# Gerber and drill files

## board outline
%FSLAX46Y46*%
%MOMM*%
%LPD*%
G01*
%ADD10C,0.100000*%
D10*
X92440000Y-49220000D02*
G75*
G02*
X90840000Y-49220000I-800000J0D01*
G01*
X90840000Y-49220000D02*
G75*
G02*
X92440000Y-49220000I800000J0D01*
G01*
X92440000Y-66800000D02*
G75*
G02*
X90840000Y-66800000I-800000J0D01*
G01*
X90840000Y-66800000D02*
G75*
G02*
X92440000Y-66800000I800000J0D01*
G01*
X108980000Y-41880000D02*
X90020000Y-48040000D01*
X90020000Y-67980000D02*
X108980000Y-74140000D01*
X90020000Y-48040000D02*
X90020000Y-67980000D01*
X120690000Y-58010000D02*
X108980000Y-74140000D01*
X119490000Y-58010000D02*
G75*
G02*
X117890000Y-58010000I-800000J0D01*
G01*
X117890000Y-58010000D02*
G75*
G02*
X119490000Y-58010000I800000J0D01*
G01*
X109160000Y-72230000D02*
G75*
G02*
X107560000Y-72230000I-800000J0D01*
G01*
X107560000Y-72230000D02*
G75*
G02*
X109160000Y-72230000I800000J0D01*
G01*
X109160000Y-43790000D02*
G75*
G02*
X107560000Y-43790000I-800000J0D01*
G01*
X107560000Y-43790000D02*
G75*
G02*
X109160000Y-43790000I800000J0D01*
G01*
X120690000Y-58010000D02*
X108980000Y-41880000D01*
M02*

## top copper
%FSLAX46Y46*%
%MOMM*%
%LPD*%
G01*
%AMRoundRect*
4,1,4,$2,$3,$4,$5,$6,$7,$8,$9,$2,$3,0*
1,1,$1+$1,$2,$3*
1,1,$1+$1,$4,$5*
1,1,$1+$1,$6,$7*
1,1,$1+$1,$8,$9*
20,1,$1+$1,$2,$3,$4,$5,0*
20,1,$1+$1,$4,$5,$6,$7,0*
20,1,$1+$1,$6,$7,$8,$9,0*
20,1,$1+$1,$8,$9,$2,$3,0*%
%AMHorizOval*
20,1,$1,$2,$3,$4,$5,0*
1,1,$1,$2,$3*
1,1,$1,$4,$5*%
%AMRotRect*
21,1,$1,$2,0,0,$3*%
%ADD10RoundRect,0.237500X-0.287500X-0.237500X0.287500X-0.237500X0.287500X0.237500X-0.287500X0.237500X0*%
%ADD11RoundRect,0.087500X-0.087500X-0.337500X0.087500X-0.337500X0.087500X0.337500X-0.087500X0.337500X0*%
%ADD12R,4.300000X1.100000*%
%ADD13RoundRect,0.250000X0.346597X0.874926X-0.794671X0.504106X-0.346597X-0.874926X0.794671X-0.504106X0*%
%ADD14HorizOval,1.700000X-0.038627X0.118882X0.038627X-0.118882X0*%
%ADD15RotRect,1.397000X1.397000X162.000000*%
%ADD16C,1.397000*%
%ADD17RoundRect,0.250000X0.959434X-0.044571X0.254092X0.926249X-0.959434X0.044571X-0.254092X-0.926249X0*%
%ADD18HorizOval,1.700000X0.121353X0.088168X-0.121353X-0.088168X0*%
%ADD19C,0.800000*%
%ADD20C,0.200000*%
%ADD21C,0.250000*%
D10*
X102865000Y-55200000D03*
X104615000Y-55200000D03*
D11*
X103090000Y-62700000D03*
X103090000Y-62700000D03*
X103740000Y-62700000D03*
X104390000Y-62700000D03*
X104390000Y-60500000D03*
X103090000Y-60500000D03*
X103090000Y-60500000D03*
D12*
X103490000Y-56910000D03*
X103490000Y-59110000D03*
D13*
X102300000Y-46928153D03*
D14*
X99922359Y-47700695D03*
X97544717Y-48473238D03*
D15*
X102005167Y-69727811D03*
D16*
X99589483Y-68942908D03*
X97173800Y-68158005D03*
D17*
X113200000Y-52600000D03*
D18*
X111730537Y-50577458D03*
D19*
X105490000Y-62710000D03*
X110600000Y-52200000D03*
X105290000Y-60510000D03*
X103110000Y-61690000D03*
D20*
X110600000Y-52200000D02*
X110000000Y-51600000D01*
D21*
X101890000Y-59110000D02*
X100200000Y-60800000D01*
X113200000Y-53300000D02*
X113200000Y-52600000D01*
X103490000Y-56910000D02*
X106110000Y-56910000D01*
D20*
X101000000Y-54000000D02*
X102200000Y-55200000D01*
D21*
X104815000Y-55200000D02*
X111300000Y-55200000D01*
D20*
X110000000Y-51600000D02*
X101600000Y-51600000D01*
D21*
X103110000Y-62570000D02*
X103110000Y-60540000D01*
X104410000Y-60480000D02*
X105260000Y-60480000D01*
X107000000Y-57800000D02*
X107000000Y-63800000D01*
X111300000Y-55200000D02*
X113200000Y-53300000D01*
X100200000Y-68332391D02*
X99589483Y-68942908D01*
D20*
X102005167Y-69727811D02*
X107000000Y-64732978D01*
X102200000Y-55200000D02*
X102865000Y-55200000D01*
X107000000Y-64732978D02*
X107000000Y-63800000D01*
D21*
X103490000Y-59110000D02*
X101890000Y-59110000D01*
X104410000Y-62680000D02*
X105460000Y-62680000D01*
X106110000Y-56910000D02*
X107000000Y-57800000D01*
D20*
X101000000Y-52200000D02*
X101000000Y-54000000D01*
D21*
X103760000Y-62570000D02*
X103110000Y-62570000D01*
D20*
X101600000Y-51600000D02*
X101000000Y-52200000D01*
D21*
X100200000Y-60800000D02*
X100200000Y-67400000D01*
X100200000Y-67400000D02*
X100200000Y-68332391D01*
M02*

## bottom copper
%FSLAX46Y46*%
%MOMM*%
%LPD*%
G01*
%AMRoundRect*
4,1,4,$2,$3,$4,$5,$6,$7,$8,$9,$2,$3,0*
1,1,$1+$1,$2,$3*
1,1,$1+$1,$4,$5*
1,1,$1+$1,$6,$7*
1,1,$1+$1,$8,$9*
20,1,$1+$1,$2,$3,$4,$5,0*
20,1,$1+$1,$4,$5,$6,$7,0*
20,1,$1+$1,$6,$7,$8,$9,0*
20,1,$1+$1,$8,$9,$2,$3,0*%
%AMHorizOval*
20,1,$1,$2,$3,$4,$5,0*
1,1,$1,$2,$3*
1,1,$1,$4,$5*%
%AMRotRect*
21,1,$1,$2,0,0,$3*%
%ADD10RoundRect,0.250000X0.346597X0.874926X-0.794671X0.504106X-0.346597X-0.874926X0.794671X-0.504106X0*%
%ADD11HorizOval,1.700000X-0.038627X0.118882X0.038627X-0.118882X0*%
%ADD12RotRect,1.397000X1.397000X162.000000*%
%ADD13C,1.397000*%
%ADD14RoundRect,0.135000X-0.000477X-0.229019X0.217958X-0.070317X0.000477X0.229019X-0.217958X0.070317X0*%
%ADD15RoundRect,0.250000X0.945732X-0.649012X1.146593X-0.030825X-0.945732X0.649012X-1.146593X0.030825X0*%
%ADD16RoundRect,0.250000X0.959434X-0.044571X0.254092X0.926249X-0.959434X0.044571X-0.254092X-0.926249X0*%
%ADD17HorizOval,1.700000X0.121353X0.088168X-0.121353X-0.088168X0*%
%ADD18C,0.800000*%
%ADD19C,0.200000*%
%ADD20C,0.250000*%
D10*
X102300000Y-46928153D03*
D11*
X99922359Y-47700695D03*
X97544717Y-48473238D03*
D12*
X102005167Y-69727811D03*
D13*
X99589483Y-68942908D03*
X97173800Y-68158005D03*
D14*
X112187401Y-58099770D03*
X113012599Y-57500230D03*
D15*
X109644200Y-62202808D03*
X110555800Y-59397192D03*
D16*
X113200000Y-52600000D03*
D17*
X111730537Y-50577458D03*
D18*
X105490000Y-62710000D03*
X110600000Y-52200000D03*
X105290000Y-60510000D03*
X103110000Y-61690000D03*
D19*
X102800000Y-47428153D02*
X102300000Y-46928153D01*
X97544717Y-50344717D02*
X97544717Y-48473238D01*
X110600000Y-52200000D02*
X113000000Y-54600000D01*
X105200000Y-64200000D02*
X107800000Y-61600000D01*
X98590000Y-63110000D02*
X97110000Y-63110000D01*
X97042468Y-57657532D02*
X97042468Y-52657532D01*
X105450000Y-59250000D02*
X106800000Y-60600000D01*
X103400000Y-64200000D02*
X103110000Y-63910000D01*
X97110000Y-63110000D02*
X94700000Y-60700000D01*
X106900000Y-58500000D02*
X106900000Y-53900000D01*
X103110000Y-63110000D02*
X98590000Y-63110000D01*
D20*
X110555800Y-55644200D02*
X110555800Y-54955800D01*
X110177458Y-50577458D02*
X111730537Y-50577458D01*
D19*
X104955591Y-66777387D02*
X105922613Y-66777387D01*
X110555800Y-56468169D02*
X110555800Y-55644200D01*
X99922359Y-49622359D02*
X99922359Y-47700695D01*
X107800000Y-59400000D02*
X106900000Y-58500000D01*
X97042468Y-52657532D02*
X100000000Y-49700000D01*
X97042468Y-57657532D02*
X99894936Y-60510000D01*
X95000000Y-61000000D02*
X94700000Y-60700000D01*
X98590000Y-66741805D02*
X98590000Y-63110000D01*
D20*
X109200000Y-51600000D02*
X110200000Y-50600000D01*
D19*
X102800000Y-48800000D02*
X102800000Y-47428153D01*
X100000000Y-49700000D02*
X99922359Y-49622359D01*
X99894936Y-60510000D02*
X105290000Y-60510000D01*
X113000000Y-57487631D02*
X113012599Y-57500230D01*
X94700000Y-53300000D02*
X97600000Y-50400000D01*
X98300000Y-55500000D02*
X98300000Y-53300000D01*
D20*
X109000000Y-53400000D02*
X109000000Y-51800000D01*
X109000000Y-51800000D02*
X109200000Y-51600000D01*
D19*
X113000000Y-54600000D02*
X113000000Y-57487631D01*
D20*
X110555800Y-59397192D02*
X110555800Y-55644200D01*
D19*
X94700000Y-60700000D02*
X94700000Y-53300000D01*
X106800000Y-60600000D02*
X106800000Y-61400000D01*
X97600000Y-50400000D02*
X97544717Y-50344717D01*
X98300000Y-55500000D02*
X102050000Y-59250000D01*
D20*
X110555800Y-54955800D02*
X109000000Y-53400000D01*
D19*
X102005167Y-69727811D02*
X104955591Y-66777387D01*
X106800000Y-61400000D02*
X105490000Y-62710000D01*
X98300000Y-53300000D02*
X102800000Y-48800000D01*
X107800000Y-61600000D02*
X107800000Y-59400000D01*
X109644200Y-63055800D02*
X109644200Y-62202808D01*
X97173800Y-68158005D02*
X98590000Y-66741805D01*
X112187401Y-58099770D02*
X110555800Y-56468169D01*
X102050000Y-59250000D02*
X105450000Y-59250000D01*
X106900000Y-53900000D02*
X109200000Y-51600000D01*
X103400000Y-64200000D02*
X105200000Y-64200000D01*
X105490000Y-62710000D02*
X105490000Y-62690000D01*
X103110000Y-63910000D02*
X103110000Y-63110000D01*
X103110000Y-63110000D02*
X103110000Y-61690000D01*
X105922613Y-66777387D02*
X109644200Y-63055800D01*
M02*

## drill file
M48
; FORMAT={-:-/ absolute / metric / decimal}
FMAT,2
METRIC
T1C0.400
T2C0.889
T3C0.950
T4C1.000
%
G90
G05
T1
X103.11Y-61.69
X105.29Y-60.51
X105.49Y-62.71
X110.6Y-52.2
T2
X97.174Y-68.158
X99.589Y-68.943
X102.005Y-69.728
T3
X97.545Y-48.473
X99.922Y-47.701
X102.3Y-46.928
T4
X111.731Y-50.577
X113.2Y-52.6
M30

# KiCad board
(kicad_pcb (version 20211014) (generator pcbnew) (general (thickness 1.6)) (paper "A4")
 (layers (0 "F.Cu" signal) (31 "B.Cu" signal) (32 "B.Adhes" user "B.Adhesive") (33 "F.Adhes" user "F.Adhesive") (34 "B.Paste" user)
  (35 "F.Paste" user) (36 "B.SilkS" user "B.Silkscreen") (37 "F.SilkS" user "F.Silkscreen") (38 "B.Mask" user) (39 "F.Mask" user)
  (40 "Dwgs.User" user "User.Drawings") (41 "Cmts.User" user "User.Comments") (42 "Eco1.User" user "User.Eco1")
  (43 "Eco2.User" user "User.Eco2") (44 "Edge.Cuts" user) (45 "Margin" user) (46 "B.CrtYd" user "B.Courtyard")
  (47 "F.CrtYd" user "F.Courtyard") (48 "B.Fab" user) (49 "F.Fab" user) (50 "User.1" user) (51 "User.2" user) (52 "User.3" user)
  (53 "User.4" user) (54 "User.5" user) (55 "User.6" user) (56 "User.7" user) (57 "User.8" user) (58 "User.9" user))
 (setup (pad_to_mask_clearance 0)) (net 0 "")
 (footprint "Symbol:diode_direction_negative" (layer "F.Cu") (at 103.8 52.65)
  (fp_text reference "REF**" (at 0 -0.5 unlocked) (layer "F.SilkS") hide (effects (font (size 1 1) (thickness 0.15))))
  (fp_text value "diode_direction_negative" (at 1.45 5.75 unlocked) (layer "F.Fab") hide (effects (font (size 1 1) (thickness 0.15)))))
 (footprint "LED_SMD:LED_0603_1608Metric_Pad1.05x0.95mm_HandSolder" (layer "F.Cu") (at 103.74 55.2)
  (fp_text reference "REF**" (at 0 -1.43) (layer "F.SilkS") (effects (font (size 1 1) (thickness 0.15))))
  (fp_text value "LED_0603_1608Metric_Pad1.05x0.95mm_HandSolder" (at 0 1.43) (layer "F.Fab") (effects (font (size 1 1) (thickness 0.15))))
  (pad "1" smd roundrect (at -0.875 0) (size 1.05 0.95) (layers "F.Cu" "F.Paste" "F.Mask") (roundrect_rratio 0.25))
  (pad "2" smd roundrect (at 0.875 0) (size 1.05 0.95) (layers "F.Cu" "F.Paste" "F.Mask") (roundrect_rratio 0.25)))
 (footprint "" (layer "F.Cu") (at 103.09 62.7)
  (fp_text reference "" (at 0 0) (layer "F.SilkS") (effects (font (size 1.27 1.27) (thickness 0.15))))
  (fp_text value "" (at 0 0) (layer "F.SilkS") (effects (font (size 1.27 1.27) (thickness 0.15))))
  (pad "1" smd roundrect (at 0 0) (size 0.35 0.85) (layers "F.Cu" "F.Paste" "F.Mask") (roundrect_rratio 0.25)))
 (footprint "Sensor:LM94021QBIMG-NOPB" (layer "F.Cu") (at 103.74 61.6)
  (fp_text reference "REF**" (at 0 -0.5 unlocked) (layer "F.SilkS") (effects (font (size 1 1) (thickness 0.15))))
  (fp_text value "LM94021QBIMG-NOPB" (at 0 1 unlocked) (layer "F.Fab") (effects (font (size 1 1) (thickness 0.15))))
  (pad "1" smd roundrect (at -0.65 1.1) (size 0.35 0.85) (layers "F.Cu" "F.Paste" "F.Mask") (roundrect_rratio 0.25))
  (pad "2" smd roundrect (at 0 1.1) (size 0.35 0.85) (layers "F.Cu" "F.Paste" "F.Mask") (roundrect_rratio 0.25))
  (pad "3" smd roundrect (at 0.65 1.1) (size 0.35 0.85) (layers "F.Cu" "F.Paste" "F.Mask") (roundrect_rratio 0.25))
  (pad "4" smd roundrect (at 0.65 -1.1) (size 0.35 0.85) (layers "F.Cu" "F.Paste" "F.Mask") (roundrect_rratio 0.25))
  (pad "5" smd roundrect (at -0.65 -1.1) (size 0.35 0.85) (layers "F.Cu" "F.Paste" "F.Mask") (roundrect_rratio 0.25)))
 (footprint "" (layer "F.Cu") (at 103.09 60.5)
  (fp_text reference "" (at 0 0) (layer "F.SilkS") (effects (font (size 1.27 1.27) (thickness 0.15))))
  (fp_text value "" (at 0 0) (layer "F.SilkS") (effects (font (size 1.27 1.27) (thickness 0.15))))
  (pad "5" smd roundrect (at 0 0) (size 0.35 0.85) (layers "F.Cu" "F.Paste" "F.Mask") (roundrect_rratio 0.25)))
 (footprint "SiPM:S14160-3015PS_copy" (layer "F.Cu") (at 103.74 58.01)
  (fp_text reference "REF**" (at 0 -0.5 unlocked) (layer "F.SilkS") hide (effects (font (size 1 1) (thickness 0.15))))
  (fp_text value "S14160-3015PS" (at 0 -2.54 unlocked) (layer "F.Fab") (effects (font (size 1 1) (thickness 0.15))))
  (pad "1" smd rect (at -0.25 -1.1) (size 4.3 1.1) (layers "F.Cu" "F.Paste" "F.Mask"))
  (pad "2" smd rect (at -0.25 1.1) (size 4.3 1.1) (layers "F.Cu" "F.Paste" "F.Mask")))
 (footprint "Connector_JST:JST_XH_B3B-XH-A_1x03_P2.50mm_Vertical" (layer "B.Cu") (at 102.3 46.928153 -162)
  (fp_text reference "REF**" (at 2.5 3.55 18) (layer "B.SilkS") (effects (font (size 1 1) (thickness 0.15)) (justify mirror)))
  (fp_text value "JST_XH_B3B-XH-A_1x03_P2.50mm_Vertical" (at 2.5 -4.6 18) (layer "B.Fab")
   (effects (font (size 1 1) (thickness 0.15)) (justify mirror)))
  (pad "1" thru_hole roundrect (at 0 0 198) (size 1.7 1.95) (drill 0.95) (layers *.Cu *.Mask) (roundrect_rratio 0.1470588235))
  (pad "2" thru_hole oval (at 2.5 0 198) (size 1.7 1.95) (drill 0.95) (layers *.Cu *.Mask))
  (pad "3" thru_hole oval (at 5 0 198) (size 1.7 1.95) (drill 0.95) (layers *.Cu *.Mask)))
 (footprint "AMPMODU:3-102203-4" (layer "B.Cu") (at 102.005167 69.727811 162)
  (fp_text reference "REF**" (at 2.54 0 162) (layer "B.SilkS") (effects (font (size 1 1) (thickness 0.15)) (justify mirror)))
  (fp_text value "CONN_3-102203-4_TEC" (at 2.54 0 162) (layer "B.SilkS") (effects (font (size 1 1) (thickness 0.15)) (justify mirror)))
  (pad "1" thru_hole rect locked (at 0 0 162) (size 1.397 1.397) (drill 0.889) (layers *.Cu *.Mask))
  (pad "2" thru_hole circle locked (at 2.54 0 162) (size 1.397 1.397) (drill 0.889) (layers *.Cu *.Mask))
  (pad "3" thru_hole circle locked (at 5.08 0 162) (size 1.397 1.397) (drill 0.889) (layers *.Cu *.Mask)))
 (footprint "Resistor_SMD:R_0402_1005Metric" (layer "B.Cu") (at 112.6 57.8 36)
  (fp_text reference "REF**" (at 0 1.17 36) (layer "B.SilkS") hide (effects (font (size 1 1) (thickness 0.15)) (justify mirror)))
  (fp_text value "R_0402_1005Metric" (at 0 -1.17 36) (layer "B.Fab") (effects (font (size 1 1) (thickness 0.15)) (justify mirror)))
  (pad "1" smd roundrect (at -0.51 0 36) (size 0.54 0.64) (layers "B.Cu" "B.Paste" "B.Mask") (roundrect_rratio 0.25))
  (pad "2" smd roundrect (at 0.51 0 36) (size 0.54 0.64) (layers "B.Cu" "B.Paste" "B.Mask") (roundrect_rratio 0.25)))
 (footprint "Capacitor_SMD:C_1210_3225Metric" (layer "B.Cu") (at 110.1 60.8 72)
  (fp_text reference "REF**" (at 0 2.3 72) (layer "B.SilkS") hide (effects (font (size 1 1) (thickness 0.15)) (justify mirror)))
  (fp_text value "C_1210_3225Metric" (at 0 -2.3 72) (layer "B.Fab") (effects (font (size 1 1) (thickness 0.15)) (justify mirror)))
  (pad "1" smd roundrect (at -1.475 0 72) (size 1.15 2.7) (layers "B.Cu" "B.Paste" "B.Mask") (roundrect_rratio 0.2173913043))
  (pad "2" smd roundrect (at 1.475 0 72) (size 1.15 2.7) (layers "B.Cu" "B.Paste" "B.Mask") (roundrect_rratio 0.2173913043)))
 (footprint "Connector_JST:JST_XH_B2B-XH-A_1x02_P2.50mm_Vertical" (layer "B.Cu") (at 113.2 52.6 126)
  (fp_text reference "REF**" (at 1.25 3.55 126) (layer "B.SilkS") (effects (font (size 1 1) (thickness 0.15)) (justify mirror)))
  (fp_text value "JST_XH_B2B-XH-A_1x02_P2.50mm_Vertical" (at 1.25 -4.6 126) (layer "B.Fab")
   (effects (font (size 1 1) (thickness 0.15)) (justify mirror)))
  (pad "1" thru_hole roundrect (at 0 0 126) (size 1.7 2) (drill 1) (layers *.Cu *.Mask) (roundrect_rratio 0.1470588235))
  (pad "2" thru_hole oval (at 2.5 0 126) (size 1.7 2) (drill 1) (layers *.Cu *.Mask)))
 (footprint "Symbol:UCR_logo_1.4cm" (layer "B.Cu") (at 113 64.5 -126)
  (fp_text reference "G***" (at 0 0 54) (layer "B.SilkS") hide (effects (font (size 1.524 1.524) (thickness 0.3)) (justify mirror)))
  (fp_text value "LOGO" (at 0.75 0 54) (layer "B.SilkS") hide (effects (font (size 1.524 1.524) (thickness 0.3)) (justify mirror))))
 (gr_circle (center 91.64 49.22) (end 92.44 49.22) (layer "Edge.Cuts") (width 0.1) (fill none))
 (gr_circle (center 91.64 66.8) (end 92.44 66.8) (layer "Edge.Cuts") (width 0.1) (fill none))
 (gr_line (start 108.98 41.88) (end 90.02 48.04) (layer "Edge.Cuts") (width 0.1))
 (gr_line (start 90.02 67.98) (end 108.98 74.14) (layer "Edge.Cuts") (width 0.1))
 (gr_line (start 90.02 48.04) (end 90.02 67.98) (layer "Edge.Cuts") (width 0.1))
 (gr_line (start 120.69 58.01) (end 108.98 74.14) (layer "Edge.Cuts") (width 0.1))
 (gr_circle (center 118.69 58.01) (end 119.49 58.01) (layer "Edge.Cuts") (width 0.1) (fill none))
 (gr_circle (center 108.36 72.23) (end 109.16 72.23) (layer "Edge.Cuts") (width 0.1) (fill none))
 (gr_circle (center 108.36 43.79) (end 109.16 43.79) (layer "Edge.Cuts") (width 0.1) (fill none))
 (gr_line (start 120.69 58.01) (end 108.98 41.88) (layer "Edge.Cuts") (width 0.1))
 (segment (start 110.6 52.2) (end 110 51.6) (width 0.2) (layer "F.Cu") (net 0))
 (segment (start 101.89 59.11) (end 100.2 60.8) (width 0.25) (layer "F.Cu") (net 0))
 (segment (start 113.2 53.3) (end 113.2 52.6) (width 0.25) (layer "F.Cu") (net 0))
 (segment (start 103.49 56.91) (end 106.11 56.91) (width 0.25) (layer "F.Cu") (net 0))
 (segment (start 101 54) (end 102.2 55.2) (width 0.2) (layer "F.Cu") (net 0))
 (segment (start 104.815 55.2) (end 111.3 55.2) (width 0.25) (layer "F.Cu") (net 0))
 (segment (start 110 51.6) (end 101.6 51.6) (width 0.2) (layer "F.Cu") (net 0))
 (segment (start 103.11 62.57) (end 103.11 60.54) (width 0.25) (layer "F.Cu") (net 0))
 (segment (start 104.41 60.48) (end 105.26 60.48) (width 0.25) (layer "F.Cu") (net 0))
 (segment (start 107 57.8) (end 107 63.8) (width 0.25) (layer "F.Cu") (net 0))
 (segment (start 111.3 55.2) (end 113.2 53.3) (width 0.25) (layer "F.Cu") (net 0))
 (segment (start 100.2 68.332391) (end 99.589483 68.942908) (width 0.25) (layer "F.Cu") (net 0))
 (segment (start 102.005167 69.727811) (end 107 64.732978) (width 0.2) (layer "F.Cu") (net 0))
 (segment (start 102.2 55.2) (end 102.865 55.2) (width 0.2) (layer "F.Cu") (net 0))
 (segment (start 107 64.732978) (end 107 63.8) (width 0.2) (layer "F.Cu") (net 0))
 (segment (start 103.49 59.11) (end 101.89 59.11) (width 0.25) (layer "F.Cu") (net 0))
 (segment (start 104.41 62.68) (end 105.46 62.68) (width 0.25) (layer "F.Cu") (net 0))
 (segment (start 106.11 56.91) (end 107 57.8) (width 0.25) (layer "F.Cu") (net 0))
 (segment (start 101 52.2) (end 101 54) (width 0.2) (layer "F.Cu") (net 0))
 (segment (start 103.76 62.57) (end 103.11 62.57) (width 0.25) (layer "F.Cu") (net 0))
 (segment (start 101.6 51.6) (end 101 52.2) (width 0.2) (layer "F.Cu") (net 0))
 (segment (start 100.2 60.8) (end 100.2 67.4) (width 0.25) (layer "F.Cu") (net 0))
 (segment (start 100.2 67.4) (end 100.2 68.332391) (width 0.25) (layer "F.Cu") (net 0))
 (via (at 105.49 62.71) (size 0.8) (drill 0.4) (layers "F.Cu" "B.Cu") (free) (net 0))
 (via (at 110.6 52.2) (size 0.8) (drill 0.4) (layers "F.Cu" "B.Cu") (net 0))
 (via (at 105.29 60.51) (size 0.8) (drill 0.4) (layers "F.Cu" "B.Cu") (free) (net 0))
 (via (at 103.11 61.69) (size 0.8) (drill 0.4) (layers "F.Cu" "B.Cu") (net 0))
 (segment (start 102.8 47.428153) (end 102.3 46.928153) (width 0.2) (layer "B.Cu") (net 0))
 (segment (start 97.544717 50.344717) (end 97.544717 48.473238) (width 0.2) (layer "B.Cu") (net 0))
 (segment (start 110.6 52.2) (end 113 54.6) (width 0.2) (layer "B.Cu") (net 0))
 (segment (start 105.2 64.2) (end 107.8 61.6) (width 0.2) (layer "B.Cu") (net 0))
 (segment (start 98.59 63.11) (end 97.11 63.11) (width 0.2) (layer "B.Cu") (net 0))
 (segment (start 97.042468 57.657532) (end 97.042468 52.657532) (width 0.2) (layer "B.Cu") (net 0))
 (segment (start 105.45 59.25) (end 106.8 60.6) (width 0.2) (layer "B.Cu") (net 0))
 (segment (start 103.4 64.2) (end 103.11 63.91) (width 0.2) (layer "B.Cu") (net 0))
 (segment (start 97.11 63.11) (end 94.7 60.7) (width 0.2) (layer "B.Cu") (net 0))
 (segment (start 106.9 58.5) (end 106.9 53.9) (width 0.2) (layer "B.Cu") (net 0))
 (segment (start 103.11 63.11) (end 98.59 63.11) (width 0.2) (layer "B.Cu") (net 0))
 (segment (start 110.5558 55.6442) (end 110.5558 54.9558) (width 0.25) (layer "B.Cu") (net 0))
 (segment (start 110.177458 50.577458) (end 111.730537 50.577458) (width 0.25) (layer "B.Cu") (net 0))
 (segment (start 104.955591 66.777387) (end 105.922613 66.777387) (width 0.2) (layer "B.Cu") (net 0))
 (segment (start 110.5558 56.468169) (end 110.5558 55.6442) (width 0.2) (layer "B.Cu") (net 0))
 (segment (start 99.922359 49.622359) (end 99.922359 47.700695) (width 0.2) (layer "B.Cu") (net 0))
 (segment (start 107.8 59.4) (end 106.9 58.5) (width 0.2) (layer "B.Cu") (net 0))
 (segment (start 97.042468 52.657532) (end 100 49.7) (width 0.2) (layer "B.Cu") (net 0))
 (segment (start 97.042468 57.657532) (end 99.894936 60.51) (width 0.2) (layer "B.Cu") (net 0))
 (segment (start 95 61) (end 94.7 60.7) (width 0.2) (layer "B.Cu") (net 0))
 (segment (start 98.59 66.741805) (end 98.59 63.11) (width 0.2) (layer "B.Cu") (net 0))
 (segment (start 109.2 51.6) (end 110.2 50.6) (width 0.25) (layer "B.Cu") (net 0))
 (segment (start 102.8 48.8) (end 102.8 47.428153) (width 0.2) (layer "B.Cu") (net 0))
 (segment (start 100 49.7) (end 99.922359 49.622359) (width 0.2) (layer "B.Cu") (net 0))
 (segment (start 99.894936 60.51) (end 105.29 60.51) (width 0.2) (layer "B.Cu") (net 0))
 (segment (start 113 57.487631) (end 113.012599 57.50023) (width 0.2) (layer "B.Cu") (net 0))
 (segment (start 94.7 53.3) (end 97.6 50.4) (width 0.2) (layer "B.Cu") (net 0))
 (segment (start 98.3 55.5) (end 98.3 53.3) (width 0.2) (layer "B.Cu") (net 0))
 (segment (start 109 53.4) (end 109 51.8) (width 0.25) (layer "B.Cu") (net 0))
 (segment (start 109 51.8) (end 109.2 51.6) (width 0.25) (layer "B.Cu") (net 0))
 (segment (start 113 54.6) (end 113 57.487631) (width 0.2) (layer "B.Cu") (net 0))
 (segment (start 110.5558 59.397192) (end 110.5558 55.6442) (width 0.25) (layer "B.Cu") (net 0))
 (segment (start 94.7 60.7) (end 94.7 53.3) (width 0.2) (layer "B.Cu") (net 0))
 (segment (start 106.8 60.6) (end 106.8 61.4) (width 0.2) (layer "B.Cu") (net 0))
 (segment (start 97.6 50.4) (end 97.544717 50.344717) (width 0.2) (layer "B.Cu") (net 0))
 (segment (start 98.3 55.5) (end 102.05 59.25) (width 0.2) (layer "B.Cu") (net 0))
 (segment (start 110.5558 54.9558) (end 109 53.4) (width 0.25) (layer "B.Cu") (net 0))
 (segment (start 102.005167 69.727811) (end 104.955591 66.777387) (width 0.2) (layer "B.Cu") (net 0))
 (segment (start 106.8 61.4) (end 105.49 62.71) (width 0.2) (layer "B.Cu") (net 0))
 (segment (start 98.3 53.3) (end 102.8 48.8) (width 0.2) (layer "B.Cu") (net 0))
 (segment (start 107.8 61.6) (end 107.8 59.4) (width 0.2) (layer "B.Cu") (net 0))
 (segment (start 109.6442 63.0558) (end 109.6442 62.202808) (width 0.2) (layer "B.Cu") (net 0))
 (segment (start 97.1738 68.158005) (end 98.59 66.741805) (width 0.2) (layer "B.Cu") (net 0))
 (segment (start 112.187401 58.09977) (end 110.5558 56.468169) (width 0.2) (layer "B.Cu") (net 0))
 (segment (start 102.05 59.25) (end 105.45 59.25) (width 0.2) (layer "B.Cu") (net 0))
 (segment (start 106.9 53.9) (end 109.2 51.6) (width 0.2) (layer "B.Cu") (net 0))
 (segment (start 103.4 64.2) (end 105.2 64.2) (width 0.2) (layer "B.Cu") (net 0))
 (segment (start 105.49 62.71) (end 105.49 62.69) (width 0.2) (layer "B.Cu") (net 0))
 (segment (start 103.11 63.91) (end 103.11 63.11) (width 0.2) (layer "B.Cu") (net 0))
 (segment (start 103.11 63.11) (end 103.11 61.69) (width 0.2) (layer "B.Cu") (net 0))
 (segment (start 105.922613 66.777387) (end 109.6442 63.0558) (width 0.2) (layer "B.Cu") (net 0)))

